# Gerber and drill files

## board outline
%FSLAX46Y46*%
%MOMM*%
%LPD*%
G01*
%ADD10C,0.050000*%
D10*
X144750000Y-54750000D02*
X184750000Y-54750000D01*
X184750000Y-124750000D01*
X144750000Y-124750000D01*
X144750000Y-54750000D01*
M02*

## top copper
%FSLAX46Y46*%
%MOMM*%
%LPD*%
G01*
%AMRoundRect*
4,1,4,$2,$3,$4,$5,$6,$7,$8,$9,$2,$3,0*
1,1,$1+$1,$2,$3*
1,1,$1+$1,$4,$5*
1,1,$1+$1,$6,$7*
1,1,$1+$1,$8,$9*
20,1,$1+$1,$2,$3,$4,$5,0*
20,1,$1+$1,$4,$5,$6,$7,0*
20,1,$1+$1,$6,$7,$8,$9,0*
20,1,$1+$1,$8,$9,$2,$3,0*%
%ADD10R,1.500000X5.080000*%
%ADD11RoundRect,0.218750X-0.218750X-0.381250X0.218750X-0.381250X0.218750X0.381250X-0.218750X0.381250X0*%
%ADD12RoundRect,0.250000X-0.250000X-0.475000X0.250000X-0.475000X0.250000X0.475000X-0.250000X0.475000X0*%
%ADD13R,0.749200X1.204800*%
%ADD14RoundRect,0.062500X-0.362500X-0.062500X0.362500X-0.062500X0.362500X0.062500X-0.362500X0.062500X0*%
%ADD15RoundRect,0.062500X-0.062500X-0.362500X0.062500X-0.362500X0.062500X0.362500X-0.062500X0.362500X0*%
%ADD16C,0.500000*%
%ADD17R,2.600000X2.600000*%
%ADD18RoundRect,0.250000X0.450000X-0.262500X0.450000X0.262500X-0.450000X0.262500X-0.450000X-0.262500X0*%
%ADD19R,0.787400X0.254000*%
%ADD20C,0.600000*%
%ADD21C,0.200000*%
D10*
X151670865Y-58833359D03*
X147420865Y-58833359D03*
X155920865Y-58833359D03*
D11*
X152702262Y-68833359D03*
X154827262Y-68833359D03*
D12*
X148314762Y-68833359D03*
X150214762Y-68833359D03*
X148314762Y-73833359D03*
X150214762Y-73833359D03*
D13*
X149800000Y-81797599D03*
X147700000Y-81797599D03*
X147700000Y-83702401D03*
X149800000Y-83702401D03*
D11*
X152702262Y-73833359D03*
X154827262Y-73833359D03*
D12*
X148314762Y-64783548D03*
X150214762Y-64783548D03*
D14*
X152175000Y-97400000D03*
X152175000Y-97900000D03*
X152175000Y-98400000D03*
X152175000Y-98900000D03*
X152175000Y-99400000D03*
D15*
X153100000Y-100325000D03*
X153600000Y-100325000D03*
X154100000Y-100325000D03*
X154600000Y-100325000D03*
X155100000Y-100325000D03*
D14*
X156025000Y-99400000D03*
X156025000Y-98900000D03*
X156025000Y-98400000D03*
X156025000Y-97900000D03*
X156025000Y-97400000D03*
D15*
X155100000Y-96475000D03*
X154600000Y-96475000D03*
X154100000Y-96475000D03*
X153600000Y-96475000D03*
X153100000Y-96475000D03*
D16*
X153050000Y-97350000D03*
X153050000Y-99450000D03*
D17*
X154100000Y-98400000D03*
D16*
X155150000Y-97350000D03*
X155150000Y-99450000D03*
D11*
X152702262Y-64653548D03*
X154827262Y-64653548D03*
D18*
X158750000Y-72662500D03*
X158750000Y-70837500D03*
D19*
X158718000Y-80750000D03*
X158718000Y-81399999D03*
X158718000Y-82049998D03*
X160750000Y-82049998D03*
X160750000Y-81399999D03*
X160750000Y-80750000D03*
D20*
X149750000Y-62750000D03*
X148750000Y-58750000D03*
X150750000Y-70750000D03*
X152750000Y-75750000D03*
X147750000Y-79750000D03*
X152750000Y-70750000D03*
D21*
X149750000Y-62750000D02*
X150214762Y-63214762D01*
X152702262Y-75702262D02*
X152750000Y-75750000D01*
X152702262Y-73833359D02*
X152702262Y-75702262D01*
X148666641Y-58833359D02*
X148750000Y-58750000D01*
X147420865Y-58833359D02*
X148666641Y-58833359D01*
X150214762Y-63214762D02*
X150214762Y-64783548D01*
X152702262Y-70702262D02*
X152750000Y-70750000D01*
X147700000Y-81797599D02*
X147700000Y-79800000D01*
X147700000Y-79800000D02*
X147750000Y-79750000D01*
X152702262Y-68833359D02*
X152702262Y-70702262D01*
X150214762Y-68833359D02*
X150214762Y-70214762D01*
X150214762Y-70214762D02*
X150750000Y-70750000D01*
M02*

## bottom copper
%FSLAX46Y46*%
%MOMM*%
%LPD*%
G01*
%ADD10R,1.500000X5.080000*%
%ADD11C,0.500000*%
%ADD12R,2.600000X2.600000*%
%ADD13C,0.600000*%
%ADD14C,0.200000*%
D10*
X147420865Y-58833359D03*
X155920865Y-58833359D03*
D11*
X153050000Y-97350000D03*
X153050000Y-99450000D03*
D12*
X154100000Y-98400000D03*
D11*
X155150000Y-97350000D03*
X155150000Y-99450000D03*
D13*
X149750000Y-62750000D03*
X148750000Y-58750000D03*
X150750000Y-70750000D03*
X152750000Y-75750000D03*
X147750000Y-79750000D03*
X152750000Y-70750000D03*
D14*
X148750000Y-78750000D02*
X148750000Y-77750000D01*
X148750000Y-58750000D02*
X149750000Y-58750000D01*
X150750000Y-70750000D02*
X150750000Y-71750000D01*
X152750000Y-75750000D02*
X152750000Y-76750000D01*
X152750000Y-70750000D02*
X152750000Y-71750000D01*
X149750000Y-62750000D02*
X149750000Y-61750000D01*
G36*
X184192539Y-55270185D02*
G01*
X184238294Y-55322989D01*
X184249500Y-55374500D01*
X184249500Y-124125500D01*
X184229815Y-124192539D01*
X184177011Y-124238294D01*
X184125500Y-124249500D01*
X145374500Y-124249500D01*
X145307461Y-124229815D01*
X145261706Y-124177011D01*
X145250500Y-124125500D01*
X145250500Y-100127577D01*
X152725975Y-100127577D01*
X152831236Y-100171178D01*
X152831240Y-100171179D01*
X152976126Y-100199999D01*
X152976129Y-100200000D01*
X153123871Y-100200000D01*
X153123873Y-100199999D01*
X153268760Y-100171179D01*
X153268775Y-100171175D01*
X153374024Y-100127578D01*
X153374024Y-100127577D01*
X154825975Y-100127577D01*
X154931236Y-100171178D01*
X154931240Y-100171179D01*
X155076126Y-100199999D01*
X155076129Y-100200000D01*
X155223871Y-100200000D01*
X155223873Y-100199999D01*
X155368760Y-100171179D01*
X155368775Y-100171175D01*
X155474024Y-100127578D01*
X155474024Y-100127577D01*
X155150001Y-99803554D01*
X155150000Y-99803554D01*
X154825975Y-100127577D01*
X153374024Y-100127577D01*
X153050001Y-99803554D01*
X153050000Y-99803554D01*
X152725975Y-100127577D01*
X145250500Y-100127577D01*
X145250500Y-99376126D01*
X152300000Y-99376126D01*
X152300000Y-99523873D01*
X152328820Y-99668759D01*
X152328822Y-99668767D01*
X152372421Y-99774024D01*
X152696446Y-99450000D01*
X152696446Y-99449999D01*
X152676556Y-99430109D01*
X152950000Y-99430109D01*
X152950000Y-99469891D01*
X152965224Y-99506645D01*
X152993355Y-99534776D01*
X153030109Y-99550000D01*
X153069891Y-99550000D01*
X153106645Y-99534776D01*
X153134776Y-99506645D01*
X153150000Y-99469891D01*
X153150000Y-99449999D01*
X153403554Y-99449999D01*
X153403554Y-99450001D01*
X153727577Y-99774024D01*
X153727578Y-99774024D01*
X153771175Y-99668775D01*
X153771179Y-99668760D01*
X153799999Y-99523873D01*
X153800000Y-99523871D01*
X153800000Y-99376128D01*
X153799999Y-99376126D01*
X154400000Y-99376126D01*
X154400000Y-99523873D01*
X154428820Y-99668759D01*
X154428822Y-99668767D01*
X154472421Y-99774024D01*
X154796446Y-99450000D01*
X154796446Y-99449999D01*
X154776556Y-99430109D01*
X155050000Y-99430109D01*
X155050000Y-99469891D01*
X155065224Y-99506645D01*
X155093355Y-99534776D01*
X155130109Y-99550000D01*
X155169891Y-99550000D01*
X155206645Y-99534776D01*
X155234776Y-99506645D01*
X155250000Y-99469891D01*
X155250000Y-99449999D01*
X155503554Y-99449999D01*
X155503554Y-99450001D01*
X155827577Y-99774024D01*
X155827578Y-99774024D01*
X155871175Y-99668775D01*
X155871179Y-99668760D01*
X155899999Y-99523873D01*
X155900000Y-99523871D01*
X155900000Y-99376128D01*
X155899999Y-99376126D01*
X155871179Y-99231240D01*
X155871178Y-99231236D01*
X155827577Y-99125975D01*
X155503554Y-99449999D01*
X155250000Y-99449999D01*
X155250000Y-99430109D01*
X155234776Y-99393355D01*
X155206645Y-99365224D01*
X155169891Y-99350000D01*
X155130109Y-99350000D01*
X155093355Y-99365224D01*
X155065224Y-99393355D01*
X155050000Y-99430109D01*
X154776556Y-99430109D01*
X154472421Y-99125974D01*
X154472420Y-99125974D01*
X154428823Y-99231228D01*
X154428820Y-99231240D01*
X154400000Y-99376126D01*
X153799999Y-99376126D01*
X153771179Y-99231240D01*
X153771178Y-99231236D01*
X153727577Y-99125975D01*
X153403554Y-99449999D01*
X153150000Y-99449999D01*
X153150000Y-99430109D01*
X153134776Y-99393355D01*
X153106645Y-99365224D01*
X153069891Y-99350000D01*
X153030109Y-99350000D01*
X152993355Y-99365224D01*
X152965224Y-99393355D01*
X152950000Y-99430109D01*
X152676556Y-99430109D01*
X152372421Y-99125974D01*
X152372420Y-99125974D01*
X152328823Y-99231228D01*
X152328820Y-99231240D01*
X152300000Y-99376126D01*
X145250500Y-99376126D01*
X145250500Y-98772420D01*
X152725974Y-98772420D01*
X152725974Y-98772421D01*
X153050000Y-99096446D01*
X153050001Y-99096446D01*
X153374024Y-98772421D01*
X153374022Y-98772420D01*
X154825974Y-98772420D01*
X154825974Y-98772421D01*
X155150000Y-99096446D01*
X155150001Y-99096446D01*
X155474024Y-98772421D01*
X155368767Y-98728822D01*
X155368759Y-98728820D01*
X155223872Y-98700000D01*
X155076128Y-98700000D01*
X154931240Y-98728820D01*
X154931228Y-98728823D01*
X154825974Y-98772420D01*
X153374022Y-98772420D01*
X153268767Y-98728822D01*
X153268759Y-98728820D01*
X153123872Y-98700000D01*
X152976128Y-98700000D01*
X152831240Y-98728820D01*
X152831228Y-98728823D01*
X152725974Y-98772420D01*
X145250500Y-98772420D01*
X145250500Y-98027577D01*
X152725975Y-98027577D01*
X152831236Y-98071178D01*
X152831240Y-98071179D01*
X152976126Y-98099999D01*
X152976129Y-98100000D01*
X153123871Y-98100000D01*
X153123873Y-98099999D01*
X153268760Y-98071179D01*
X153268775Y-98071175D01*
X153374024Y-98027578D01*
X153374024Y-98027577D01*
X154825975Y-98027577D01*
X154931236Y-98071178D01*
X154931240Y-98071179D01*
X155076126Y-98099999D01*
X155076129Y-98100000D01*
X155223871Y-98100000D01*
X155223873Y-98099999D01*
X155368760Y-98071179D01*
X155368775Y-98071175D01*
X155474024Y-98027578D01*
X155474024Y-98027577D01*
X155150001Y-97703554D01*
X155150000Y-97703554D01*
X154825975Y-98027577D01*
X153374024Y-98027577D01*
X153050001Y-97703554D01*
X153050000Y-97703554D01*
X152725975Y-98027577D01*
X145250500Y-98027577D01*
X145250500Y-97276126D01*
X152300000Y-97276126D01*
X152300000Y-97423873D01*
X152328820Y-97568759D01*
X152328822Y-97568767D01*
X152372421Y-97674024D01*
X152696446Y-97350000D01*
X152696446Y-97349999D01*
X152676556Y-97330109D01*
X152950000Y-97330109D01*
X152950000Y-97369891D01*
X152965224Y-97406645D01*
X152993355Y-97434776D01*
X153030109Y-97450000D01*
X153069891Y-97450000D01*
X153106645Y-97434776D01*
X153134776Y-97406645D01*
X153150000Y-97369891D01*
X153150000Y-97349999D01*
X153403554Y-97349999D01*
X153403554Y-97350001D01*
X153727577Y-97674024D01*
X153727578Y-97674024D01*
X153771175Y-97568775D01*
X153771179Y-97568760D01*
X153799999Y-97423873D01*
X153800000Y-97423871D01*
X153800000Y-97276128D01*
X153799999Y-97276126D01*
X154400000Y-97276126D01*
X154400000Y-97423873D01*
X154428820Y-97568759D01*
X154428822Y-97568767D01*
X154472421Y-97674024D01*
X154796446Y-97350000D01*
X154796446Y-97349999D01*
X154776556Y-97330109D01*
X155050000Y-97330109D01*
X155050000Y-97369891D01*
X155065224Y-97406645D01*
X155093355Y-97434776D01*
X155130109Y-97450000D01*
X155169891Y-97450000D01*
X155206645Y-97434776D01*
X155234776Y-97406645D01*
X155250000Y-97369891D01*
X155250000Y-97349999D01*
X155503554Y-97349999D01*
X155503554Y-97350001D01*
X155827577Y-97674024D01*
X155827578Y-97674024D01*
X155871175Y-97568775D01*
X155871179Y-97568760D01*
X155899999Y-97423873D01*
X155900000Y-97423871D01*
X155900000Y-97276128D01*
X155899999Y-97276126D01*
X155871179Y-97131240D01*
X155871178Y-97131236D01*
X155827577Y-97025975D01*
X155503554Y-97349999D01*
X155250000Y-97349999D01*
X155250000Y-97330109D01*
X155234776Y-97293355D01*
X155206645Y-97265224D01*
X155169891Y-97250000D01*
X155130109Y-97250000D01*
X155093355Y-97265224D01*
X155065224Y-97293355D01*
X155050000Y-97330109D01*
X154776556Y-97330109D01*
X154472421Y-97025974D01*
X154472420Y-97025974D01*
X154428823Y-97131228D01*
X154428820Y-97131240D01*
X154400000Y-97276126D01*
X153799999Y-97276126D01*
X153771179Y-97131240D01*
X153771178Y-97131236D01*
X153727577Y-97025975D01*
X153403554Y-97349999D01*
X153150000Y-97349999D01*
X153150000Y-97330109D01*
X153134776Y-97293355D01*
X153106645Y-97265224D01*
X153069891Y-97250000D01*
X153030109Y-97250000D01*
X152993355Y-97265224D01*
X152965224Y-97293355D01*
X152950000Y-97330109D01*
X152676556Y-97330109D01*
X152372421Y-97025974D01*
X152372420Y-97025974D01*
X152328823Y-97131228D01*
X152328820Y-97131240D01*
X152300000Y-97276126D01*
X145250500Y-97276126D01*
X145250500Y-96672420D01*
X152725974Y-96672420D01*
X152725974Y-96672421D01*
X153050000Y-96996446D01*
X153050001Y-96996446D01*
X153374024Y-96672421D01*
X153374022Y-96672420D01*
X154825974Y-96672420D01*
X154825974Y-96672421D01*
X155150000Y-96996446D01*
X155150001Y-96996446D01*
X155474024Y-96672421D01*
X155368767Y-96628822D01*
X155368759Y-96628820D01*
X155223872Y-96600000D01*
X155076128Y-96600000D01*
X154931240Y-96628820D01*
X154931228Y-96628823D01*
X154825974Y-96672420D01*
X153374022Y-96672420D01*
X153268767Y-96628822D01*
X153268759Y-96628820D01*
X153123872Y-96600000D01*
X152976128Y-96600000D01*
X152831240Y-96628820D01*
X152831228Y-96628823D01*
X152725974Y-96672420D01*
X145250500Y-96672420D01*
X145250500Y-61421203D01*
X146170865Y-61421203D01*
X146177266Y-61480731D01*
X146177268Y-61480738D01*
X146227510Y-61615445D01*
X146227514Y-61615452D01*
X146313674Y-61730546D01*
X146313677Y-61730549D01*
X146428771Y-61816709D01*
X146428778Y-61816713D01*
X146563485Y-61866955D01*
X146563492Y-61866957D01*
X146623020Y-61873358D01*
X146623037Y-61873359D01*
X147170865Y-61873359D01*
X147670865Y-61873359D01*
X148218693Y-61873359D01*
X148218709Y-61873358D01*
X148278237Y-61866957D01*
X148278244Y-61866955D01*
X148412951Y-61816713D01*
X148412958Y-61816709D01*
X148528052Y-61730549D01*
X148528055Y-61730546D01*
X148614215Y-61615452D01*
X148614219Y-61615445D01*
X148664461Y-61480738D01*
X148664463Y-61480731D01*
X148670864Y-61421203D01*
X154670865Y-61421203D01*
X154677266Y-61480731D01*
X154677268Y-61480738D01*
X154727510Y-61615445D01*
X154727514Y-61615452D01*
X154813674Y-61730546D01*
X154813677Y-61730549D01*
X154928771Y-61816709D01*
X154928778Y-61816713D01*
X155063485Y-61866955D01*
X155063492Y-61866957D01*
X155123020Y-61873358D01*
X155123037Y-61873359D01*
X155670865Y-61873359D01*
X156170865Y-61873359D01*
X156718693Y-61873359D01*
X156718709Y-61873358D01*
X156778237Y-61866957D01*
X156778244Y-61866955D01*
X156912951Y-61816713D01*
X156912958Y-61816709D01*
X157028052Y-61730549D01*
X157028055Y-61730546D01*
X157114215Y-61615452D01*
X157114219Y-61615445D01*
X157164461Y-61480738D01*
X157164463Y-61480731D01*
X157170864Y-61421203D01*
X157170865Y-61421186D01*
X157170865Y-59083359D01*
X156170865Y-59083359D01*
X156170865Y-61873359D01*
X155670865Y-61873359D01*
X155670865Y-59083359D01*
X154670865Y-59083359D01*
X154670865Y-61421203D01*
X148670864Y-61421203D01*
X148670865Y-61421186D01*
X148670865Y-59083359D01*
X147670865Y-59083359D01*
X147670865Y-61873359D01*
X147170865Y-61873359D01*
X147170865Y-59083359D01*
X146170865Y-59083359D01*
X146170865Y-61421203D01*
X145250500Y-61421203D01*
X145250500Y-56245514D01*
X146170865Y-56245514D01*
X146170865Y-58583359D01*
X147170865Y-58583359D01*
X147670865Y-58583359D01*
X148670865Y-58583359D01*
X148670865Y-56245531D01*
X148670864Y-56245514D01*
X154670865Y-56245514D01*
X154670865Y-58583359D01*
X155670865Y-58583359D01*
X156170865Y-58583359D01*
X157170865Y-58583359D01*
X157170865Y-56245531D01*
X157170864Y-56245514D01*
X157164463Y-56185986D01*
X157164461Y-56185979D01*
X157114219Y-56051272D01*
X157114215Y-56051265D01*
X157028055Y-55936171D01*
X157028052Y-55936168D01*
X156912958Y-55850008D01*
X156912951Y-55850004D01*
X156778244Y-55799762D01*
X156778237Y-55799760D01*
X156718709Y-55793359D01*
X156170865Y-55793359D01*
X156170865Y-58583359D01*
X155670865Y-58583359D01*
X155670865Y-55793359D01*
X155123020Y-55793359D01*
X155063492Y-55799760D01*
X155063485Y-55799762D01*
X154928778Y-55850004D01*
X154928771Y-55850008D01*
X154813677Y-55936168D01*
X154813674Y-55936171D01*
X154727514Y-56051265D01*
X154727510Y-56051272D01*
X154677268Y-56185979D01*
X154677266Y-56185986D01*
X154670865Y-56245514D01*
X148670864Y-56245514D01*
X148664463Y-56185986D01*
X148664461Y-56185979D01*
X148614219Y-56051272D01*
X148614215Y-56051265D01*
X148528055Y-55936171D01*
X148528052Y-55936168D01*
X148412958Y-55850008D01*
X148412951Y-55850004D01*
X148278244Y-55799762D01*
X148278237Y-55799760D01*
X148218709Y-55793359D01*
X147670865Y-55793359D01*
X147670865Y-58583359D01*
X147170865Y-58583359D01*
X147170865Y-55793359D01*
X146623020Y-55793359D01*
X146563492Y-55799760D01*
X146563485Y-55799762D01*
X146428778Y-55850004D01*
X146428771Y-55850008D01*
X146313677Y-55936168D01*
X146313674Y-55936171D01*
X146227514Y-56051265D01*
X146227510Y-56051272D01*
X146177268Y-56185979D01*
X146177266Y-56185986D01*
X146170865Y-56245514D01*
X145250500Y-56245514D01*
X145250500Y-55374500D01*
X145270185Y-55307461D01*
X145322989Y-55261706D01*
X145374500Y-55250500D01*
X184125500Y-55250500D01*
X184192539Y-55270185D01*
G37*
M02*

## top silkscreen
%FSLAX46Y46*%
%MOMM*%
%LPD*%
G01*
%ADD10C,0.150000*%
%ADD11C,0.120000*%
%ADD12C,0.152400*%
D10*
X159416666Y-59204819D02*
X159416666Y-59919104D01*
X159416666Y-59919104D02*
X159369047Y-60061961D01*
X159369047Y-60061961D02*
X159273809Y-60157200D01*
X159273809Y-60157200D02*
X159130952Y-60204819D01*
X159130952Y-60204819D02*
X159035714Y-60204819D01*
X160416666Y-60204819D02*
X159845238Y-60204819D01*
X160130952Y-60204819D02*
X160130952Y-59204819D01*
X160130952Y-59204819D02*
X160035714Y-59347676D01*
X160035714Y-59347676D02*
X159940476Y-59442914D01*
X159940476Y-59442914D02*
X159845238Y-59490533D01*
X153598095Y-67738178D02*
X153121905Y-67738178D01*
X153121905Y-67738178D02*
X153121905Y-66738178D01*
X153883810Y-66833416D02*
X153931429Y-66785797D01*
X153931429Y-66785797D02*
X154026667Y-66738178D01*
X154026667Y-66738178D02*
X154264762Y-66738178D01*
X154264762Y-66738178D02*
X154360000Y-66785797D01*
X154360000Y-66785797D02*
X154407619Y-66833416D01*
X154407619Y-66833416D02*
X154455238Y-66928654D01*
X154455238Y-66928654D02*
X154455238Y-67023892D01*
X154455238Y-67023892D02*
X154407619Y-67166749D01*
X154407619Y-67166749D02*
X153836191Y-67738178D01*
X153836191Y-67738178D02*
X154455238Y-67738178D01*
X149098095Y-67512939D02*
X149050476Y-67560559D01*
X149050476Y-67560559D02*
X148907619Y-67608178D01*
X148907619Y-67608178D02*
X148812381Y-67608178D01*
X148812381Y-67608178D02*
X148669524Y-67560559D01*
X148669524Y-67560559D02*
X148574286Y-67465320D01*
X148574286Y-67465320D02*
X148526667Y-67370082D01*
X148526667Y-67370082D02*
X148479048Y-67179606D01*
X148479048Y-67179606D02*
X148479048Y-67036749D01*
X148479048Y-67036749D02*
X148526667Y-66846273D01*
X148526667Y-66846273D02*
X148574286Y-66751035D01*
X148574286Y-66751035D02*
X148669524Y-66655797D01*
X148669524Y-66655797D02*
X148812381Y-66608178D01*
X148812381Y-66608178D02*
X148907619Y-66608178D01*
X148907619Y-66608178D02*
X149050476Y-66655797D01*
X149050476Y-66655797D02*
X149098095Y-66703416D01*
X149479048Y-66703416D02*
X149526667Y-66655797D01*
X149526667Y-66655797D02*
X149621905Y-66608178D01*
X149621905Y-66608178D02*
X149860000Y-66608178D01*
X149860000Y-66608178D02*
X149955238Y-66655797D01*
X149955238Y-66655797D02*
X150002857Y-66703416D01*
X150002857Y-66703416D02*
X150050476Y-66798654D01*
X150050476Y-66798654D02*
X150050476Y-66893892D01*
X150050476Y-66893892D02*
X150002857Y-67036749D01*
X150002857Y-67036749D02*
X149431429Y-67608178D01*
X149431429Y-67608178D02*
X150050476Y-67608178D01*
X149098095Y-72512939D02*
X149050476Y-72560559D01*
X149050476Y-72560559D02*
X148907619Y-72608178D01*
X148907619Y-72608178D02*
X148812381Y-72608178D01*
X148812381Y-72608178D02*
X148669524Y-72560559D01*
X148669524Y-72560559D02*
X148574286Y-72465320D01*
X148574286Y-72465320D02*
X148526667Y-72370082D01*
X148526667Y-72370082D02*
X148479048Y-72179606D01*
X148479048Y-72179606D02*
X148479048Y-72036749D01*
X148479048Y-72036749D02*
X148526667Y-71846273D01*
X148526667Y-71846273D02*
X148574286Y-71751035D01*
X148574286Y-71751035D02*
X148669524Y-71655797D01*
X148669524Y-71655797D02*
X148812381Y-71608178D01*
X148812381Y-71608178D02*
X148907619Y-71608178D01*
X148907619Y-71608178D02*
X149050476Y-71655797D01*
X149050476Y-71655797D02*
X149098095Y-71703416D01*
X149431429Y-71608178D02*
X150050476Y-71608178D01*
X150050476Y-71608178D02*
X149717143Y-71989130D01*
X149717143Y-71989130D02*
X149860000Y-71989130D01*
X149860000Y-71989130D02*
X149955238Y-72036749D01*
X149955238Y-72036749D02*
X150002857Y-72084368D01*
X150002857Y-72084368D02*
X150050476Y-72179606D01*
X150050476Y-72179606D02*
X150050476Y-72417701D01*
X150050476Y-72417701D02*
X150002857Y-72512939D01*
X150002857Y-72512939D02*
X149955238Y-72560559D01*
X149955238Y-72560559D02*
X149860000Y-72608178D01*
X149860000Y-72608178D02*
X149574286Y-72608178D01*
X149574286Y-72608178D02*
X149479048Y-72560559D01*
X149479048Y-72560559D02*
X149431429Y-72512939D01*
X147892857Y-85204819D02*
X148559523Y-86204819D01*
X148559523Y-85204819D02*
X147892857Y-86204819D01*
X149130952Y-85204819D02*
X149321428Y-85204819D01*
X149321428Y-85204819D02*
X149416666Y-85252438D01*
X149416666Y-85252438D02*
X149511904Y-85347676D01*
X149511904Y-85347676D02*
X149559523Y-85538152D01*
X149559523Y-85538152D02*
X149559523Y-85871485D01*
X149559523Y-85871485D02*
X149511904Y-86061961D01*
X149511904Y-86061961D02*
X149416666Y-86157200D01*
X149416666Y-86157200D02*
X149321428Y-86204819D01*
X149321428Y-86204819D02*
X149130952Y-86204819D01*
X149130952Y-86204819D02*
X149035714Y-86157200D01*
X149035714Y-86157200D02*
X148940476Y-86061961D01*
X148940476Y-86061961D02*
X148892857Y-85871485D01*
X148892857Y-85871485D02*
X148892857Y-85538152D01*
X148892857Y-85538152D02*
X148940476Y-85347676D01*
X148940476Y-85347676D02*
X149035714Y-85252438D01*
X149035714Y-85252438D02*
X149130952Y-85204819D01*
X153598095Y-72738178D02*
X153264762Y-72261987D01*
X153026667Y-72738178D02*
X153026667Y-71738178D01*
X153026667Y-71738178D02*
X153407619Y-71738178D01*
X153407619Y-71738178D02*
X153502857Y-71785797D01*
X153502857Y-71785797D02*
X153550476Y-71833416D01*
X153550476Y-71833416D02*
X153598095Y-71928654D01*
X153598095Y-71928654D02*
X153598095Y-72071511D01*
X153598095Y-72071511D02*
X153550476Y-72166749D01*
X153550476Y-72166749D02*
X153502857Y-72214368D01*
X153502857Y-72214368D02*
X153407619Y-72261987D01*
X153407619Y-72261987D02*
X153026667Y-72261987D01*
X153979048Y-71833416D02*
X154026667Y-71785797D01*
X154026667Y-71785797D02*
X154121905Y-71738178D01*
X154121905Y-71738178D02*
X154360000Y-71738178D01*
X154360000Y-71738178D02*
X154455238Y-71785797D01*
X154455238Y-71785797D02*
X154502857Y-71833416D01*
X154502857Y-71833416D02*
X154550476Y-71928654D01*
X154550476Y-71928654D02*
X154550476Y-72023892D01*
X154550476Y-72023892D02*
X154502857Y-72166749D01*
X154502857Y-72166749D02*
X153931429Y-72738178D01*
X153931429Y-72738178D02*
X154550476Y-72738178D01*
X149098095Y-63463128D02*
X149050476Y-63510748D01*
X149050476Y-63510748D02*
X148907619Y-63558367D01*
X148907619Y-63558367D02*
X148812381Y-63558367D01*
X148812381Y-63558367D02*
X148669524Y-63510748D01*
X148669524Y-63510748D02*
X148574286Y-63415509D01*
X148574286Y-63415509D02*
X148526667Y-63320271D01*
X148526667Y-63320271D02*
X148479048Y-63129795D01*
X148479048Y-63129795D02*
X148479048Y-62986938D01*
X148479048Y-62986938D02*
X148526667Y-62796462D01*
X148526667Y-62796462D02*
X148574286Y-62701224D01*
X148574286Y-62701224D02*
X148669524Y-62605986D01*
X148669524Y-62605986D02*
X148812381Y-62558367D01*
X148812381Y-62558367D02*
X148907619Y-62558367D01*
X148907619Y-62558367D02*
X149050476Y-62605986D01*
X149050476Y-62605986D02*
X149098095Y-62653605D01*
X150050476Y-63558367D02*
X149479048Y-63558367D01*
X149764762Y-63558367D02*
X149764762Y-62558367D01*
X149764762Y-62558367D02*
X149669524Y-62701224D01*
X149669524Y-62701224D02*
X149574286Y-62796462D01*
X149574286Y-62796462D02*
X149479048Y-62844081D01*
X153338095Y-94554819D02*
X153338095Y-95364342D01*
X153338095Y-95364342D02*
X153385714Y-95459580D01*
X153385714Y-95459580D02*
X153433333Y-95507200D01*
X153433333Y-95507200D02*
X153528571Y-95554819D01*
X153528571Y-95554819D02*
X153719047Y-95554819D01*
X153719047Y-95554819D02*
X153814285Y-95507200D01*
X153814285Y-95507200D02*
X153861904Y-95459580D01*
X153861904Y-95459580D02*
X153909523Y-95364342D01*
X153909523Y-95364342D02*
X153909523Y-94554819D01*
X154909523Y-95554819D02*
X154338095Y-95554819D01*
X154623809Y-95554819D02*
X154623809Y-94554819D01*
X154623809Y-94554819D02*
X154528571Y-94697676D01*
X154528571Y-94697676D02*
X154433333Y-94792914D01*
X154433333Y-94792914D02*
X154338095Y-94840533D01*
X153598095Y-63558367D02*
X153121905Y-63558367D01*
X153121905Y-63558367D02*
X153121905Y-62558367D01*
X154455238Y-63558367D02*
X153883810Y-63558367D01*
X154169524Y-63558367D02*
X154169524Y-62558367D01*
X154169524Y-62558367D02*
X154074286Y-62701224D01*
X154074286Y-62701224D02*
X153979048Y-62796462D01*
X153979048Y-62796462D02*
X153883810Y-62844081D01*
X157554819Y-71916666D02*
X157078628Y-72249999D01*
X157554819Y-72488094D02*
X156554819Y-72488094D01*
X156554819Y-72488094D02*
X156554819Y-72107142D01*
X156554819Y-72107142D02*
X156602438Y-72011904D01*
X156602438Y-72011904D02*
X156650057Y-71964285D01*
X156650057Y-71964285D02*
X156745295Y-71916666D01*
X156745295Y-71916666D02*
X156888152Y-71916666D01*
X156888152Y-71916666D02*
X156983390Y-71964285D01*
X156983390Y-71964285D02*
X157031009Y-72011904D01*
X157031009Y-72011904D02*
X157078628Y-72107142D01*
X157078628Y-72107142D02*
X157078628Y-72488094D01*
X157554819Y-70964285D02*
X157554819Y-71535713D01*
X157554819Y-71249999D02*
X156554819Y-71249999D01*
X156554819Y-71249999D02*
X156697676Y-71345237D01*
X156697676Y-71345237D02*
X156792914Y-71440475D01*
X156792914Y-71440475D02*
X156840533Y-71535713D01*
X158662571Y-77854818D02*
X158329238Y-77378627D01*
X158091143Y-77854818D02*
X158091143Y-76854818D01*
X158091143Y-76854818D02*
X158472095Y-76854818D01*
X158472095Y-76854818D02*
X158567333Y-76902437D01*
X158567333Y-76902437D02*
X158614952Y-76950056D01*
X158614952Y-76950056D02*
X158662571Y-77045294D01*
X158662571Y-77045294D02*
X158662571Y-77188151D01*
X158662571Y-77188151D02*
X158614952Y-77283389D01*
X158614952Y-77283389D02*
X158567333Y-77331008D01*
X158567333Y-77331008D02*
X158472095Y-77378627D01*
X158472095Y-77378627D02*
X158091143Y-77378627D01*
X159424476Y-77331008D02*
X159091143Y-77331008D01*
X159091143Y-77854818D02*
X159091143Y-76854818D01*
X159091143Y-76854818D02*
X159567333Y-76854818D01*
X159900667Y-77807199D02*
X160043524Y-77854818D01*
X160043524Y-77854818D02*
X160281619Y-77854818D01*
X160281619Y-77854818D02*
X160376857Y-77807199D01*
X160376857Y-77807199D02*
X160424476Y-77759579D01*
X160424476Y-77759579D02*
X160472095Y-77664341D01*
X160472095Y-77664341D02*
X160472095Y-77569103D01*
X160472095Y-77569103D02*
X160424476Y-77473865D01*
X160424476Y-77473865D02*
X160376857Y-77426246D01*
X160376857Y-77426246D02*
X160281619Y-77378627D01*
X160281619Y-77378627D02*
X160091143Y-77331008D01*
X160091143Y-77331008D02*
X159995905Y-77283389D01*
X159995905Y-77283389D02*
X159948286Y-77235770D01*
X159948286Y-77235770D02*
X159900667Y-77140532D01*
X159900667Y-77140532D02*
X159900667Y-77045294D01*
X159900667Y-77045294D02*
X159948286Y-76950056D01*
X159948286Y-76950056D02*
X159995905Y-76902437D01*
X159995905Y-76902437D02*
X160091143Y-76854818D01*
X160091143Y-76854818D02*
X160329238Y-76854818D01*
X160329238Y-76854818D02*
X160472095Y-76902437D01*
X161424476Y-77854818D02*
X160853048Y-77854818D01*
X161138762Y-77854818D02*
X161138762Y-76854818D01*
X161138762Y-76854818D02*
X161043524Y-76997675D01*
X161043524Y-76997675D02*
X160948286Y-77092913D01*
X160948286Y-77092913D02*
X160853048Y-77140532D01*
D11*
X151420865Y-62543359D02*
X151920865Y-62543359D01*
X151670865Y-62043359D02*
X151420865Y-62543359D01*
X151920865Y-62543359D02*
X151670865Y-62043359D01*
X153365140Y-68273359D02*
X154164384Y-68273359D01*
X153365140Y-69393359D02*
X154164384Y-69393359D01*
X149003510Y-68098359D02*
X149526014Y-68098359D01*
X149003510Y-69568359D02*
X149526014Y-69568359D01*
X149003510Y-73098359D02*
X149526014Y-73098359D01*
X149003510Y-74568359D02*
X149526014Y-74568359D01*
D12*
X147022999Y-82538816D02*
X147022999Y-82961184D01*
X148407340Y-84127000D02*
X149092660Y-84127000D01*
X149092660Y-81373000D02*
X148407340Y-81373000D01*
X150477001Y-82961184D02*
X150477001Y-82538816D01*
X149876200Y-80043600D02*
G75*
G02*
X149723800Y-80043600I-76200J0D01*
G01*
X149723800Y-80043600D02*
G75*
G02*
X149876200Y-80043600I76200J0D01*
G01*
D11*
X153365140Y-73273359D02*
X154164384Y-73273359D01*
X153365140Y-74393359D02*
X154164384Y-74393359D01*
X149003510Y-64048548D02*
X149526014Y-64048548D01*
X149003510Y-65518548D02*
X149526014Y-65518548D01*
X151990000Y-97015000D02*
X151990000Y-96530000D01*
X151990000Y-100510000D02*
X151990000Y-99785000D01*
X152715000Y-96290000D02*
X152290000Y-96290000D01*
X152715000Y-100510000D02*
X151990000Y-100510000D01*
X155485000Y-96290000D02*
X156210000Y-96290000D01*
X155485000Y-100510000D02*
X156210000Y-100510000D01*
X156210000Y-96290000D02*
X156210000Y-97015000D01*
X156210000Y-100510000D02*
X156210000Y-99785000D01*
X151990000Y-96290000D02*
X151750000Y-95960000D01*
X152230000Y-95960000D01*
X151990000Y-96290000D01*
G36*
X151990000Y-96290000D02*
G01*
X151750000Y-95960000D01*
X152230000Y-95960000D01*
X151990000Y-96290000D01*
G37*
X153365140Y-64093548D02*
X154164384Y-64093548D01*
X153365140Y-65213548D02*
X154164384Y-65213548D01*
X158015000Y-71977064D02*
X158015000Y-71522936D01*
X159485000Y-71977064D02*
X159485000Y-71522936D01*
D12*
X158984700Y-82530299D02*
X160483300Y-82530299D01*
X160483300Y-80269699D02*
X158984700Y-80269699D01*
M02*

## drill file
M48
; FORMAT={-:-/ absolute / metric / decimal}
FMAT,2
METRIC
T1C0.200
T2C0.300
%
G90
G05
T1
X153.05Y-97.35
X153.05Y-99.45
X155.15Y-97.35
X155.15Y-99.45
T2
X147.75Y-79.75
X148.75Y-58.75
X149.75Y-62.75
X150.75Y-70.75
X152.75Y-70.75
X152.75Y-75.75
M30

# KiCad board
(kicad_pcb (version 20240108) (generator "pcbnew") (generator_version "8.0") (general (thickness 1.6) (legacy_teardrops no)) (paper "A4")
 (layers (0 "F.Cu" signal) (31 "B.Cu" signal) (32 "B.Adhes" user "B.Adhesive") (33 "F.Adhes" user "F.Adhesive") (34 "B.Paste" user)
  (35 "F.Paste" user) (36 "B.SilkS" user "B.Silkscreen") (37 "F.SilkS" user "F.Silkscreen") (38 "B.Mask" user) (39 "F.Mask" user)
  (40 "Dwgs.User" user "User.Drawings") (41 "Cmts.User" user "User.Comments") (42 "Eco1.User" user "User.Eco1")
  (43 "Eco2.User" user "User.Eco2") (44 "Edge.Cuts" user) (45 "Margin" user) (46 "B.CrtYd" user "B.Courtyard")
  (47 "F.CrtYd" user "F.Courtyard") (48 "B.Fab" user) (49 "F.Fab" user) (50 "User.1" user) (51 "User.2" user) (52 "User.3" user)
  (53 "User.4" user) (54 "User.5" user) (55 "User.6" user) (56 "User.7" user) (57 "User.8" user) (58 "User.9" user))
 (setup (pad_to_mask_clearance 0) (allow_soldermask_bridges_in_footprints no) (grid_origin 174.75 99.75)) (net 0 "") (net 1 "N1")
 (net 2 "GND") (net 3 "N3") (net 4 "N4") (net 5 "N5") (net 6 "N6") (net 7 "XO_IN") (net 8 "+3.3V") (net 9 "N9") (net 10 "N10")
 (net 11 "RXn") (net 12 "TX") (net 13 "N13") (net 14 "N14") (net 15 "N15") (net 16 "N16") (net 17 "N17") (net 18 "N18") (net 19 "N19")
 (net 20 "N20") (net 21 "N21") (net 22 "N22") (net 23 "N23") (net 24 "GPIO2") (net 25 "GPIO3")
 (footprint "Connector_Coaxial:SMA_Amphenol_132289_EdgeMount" (layer "F.Cu") (at 151.670865 58.833359 90)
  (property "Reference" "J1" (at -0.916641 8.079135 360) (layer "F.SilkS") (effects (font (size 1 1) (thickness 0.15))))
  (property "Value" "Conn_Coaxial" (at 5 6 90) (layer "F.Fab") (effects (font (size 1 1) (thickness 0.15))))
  (fp_line (start -3.71 -0.25) (end -3.71 0.25) (stroke (width 0.12) (type solid)) (layer "F.SilkS"))
  (fp_line (start -3.21 0) (end -3.71 -0.25) (stroke (width 0.12) (type solid)) (layer "F.SilkS"))
  (fp_line (start -3.71 0.25) (end -3.21 0) (stroke (width 0.12) (type solid)) (layer "F.SilkS"))
  (pad "1" smd rect (at 0 0 180) (size 1.5 5.08) (layers "F.Cu" "F.Paste" "F.Mask") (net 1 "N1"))
  (pad "2" smd rect (at 0 -4.25 180) (size 1.5 5.08) (layers "F.Cu" "F.Paste" "F.Mask") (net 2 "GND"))
  (pad "2" smd rect (at 0 -4.25 180) (size 1.5 5.08) (layers "B.Cu" "B.Paste" "B.Mask") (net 2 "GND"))
  (pad "2" smd rect (at 0 4.25 180) (size 1.5 5.08) (layers "F.Cu" "F.Paste" "F.Mask") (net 2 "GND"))
  (pad "2" smd rect (at 0 4.25 180) (size 1.5 5.08) (layers "B.Cu" "B.Paste" "B.Mask") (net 2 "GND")))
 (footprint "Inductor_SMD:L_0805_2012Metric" (layer "F.Cu") (at 153.764762 68.833359)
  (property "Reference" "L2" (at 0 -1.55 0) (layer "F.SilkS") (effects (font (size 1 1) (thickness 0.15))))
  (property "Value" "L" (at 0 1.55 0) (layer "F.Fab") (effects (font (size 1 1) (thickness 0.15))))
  (fp_line (start -0.399622 -0.56) (end 0.399622 -0.56) (stroke (width 0.12) (type solid)) (layer "F.SilkS"))
  (fp_line (start -0.399622 0.56) (end 0.399622 0.56) (stroke (width 0.12) (type solid)) (layer "F.SilkS"))
  (pad "1" smd roundrect (at -1.0625 0) (size 0.875 1.2) (layers "F.Cu" "F.Paste" "F.Mask") (roundrect_rratio 0.25) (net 2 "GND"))
  (pad "2" smd roundrect (at 1.0625 0) (size 0.875 1.2) (layers "F.Cu" "F.Paste" "F.Mask") (roundrect_rratio 0.25) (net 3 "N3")))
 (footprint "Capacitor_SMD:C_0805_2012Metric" (layer "F.Cu") (at 149.264762 68.833359)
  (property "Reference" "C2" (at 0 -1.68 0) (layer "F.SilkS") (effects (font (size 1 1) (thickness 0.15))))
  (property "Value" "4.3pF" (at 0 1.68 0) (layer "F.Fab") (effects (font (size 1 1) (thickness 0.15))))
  (fp_line (start -0.261252 -0.735) (end 0.261252 -0.735) (stroke (width 0.12) (type solid)) (layer "F.SilkS"))
  (fp_line (start -0.261252 0.735) (end 0.261252 0.735) (stroke (width 0.12) (type solid)) (layer "F.SilkS"))
  (pad "1" smd roundrect (at -0.95 0) (size 1 1.45) (layers "F.Cu" "F.Paste" "F.Mask") (roundrect_rratio 0.25) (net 1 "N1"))
  (pad "2" smd roundrect (at 0.95 0) (size 1 1.45) (layers "F.Cu" "F.Paste" "F.Mask") (roundrect_rratio 0.25) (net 2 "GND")))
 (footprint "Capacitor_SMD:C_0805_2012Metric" (layer "F.Cu") (at 149.264762 73.833359)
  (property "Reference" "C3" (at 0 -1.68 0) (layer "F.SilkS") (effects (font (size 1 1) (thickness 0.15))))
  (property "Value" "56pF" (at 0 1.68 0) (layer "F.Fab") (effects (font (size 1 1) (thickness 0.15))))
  (fp_line (start -0.261252 -0.735) (end 0.261252 -0.735) (stroke (width 0.12) (type solid)) (layer "F.SilkS"))
  (fp_line (start -0.261252 0.735) (end 0.261252 0.735) (stroke (width 0.12) (type solid)) (layer "F.SilkS"))
  (pad "1" smd roundrect (at -0.95 0) (size 1 1.45) (layers "F.Cu" "F.Paste" "F.Mask") (roundrect_rratio 0.25) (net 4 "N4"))
  (pad "2" smd roundrect (at 0.95 0) (size 1 1.45) (layers "F.Cu" "F.Paste" "F.Mask") (roundrect_rratio 0.25) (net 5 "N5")))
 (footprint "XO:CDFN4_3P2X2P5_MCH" (layer "F.Cu") (at 148.75 82.75 -90)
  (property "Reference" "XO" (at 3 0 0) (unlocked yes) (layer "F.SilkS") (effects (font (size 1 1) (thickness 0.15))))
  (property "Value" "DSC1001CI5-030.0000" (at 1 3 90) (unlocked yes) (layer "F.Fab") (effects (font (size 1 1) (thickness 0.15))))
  (fp_line (start -0.211184 1.727001) (end 0.211184 1.727001) (stroke (width 0.1524) (type solid)) (layer "F.SilkS"))
  (fp_line (start 1.377 0.34266) (end 1.377 -0.34266) (stroke (width 0.1524) (type solid)) (layer "F.SilkS"))
  (fp_line (start -1.377 -0.34266) (end -1.377 0.34266) (stroke (width 0.1524) (type solid)) (layer "F.SilkS"))
  (fp_line (start 0.211184 -1.727001) (end -0.211184 -1.727001) (stroke (width 0.1524) (type solid)) (layer "F.SilkS"))
  (fp_circle (center -2.7064 -1.05) (end -2.6302 -1.05) (stroke (width 0.1524) (type solid)) (fill none) (layer "F.SilkS"))
  (pad "1" smd rect (at -0.952401 -1.05 270) (size 1.2048 0.7492) (layers "F.Cu" "F.Paste" "F.Mask") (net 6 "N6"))
  (pad "2" smd rect (at -0.952401 1.05 270) (size 1.2048 0.7492) (layers "F.Cu" "F.Paste" "F.Mask") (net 2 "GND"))
  (pad "3" smd rect (at 0.952401 1.05 270) (size 1.2048 0.7492) (layers "F.Cu" "F.Paste" "F.Mask") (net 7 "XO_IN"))
  (pad "4" smd rect (at 0.952401 -1.05 270) (size 1.2048 0.7492) (layers "F.Cu" "F.Paste" "F.Mask") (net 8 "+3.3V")))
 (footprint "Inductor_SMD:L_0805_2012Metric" (layer "F.Cu") (at 153.764762 73.833359)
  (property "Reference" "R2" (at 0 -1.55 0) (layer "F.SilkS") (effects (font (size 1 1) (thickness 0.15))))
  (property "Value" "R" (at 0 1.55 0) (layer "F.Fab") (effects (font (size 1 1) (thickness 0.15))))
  (fp_line (start -0.399622 -0.56) (end 0.399622 -0.56) (stroke (width 0.12) (type solid)) (layer "F.SilkS"))
  (fp_line (start -0.399622 0.56) (end 0.399622 0.56) (stroke (width 0.12) (type solid)) (layer "F.SilkS"))
  (pad "1" smd roundrect (at -1.0625 0) (size 0.875 1.2) (layers "F.Cu" "F.Paste" "F.Mask") (roundrect_rratio 0.25) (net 2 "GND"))
  (pad "2" smd roundrect (at 1.0625 0) (size 0.875 1.2) (layers "F.Cu" "F.Paste" "F.Mask") (roundrect_rratio 0.25) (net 4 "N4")))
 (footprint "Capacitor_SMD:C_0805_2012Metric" (layer "F.Cu") (at 149.264762 64.783548)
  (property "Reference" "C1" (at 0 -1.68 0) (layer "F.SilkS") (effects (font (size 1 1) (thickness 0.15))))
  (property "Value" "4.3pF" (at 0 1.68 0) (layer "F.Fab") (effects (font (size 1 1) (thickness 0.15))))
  (fp_line (start -0.261252 -0.735) (end 0.261252 -0.735) (stroke (width 0.12) (type solid)) (layer "F.SilkS"))
  (fp_line (start -0.261252 0.735) (end 0.261252 0.735) (stroke (width 0.12) (type solid)) (layer "F.SilkS"))
  (pad "1" smd roundrect (at -0.95 0) (size 1 1.45) (layers "F.Cu" "F.Paste" "F.Mask") (roundrect_rratio 0.25) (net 5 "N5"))
  (pad "2" smd roundrect (at 0.95 0) (size 1 1.45) (layers "F.Cu" "F.Paste" "F.Mask") (roundrect_rratio 0.25) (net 2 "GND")))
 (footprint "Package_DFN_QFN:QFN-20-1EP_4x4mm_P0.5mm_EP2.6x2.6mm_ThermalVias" (layer "F.Cu") (at 154.1 98.4)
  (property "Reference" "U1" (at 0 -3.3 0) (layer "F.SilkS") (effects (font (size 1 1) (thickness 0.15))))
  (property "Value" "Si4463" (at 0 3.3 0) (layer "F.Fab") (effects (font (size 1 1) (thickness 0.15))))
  (fp_line (start -2.11 -1.385) (end -2.11 -1.87) (stroke (width 0.12) (type solid)) (layer "F.SilkS"))
  (fp_line (start -2.11 2.11) (end -2.11 1.385) (stroke (width 0.12) (type solid)) (layer "F.SilkS"))
  (fp_line (start -1.385 -2.11) (end -1.81 -2.11) (stroke (width 0.12) (type solid)) (layer "F.SilkS"))
  (fp_line (start -1.385 2.11) (end -2.11 2.11) (stroke (width 0.12) (type solid)) (layer "F.SilkS"))
  (fp_line (start 1.385 -2.11) (end 2.11 -2.11) (stroke (width 0.12) (type solid)) (layer "F.SilkS"))
  (fp_line (start 1.385 2.11) (end 2.11 2.11) (stroke (width 0.12) (type solid)) (layer "F.SilkS"))
  (fp_line (start 2.11 -2.11) (end 2.11 -1.385) (stroke (width 0.12) (type solid)) (layer "F.SilkS"))
  (fp_line (start 2.11 2.11) (end 2.11 1.385) (stroke (width 0.12) (type solid)) (layer "F.SilkS"))
  (fp_poly
   (pts (xy -2.11 -2.11) (xy -2.35 -2.44) (xy -1.87 -2.44) (xy -2.11 -2.11)) (stroke (width 0.12) (type solid)) (fill solid)
   (layer "F.SilkS"))
  (pad "" smd roundrect (at -0.65 -0.65) (size 1.13 1.13) (layers "F.Paste") (roundrect_rratio 0.221239))
  (pad "" smd roundrect (at -0.65 0.65) (size 1.13 1.13) (layers "F.Paste") (roundrect_rratio 0.221239))
  (pad "" smd roundrect (at 0.65 -0.65) (size 1.13 1.13) (layers "F.Paste") (roundrect_rratio 0.221239))
  (pad "" smd roundrect (at 0.65 0.65) (size 1.13 1.13) (layers "F.Paste") (roundrect_rratio 0.221239))
  (pad "1" smd roundrect (at -1.925 -1) (size 0.85 0.25) (layers "F.Cu" "F.Paste" "F.Mask") (roundrect_rratio 0.25) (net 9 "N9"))
  (pad "2" smd roundrect (at -1.925 -0.5) (size 0.85 0.25) (layers "F.Cu" "F.Paste" "F.Mask") (roundrect_rratio 0.25) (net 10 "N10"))
  (pad "3" smd roundrect (at -1.925 0) (size 0.85 0.25) (layers "F.Cu" "F.Paste" "F.Mask") (roundrect_rratio 0.25) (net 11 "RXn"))
  (pad "4" smd roundrect (at -1.925 0.5) (size 0.85 0.25) (layers "F.Cu" "F.Paste" "F.Mask") (roundrect_rratio 0.25) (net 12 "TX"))
  (pad "5" smd roundrect (at -1.925 1) (size 0.85 0.25) (layers "F.Cu" "F.Paste" "F.Mask") (roundrect_rratio 0.25) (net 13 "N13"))
  (pad "6" smd roundrect (at -1 1.925) (size 0.25 0.85) (layers "F.Cu" "F.Paste" "F.Mask") (roundrect_rratio 0.25) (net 8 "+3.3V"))
  (pad "7" smd roundrect (at -0.5 1.925) (size 0.25 0.85) (layers "F.Cu" "F.Paste" "F.Mask") (roundrect_rratio 0.25) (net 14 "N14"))
  (pad "8" smd roundrect (at 0 1.925) (size 0.25 0.85) (layers "F.Cu" "F.Paste" "F.Mask") (roundrect_rratio 0.25) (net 8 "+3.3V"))
  (pad "9" smd roundrect (at 0.5 1.925) (size 0.25 0.85) (layers "F.Cu" "F.Paste" "F.Mask") (roundrect_rratio 0.25) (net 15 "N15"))
  (pad "10" smd roundrect (at 1 1.925) (size 0.25 0.85) (layers "F.Cu" "F.Paste" "F.Mask") (roundrect_rratio 0.25) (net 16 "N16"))
  (pad "11" smd roundrect (at 1.925 1) (size 0.85 0.25) (layers "F.Cu" "F.Paste" "F.Mask") (roundrect_rratio 0.25) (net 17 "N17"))
  (pad "12" smd roundrect (at 1.925 0.5) (size 0.85 0.25) (layers "F.Cu" "F.Paste" "F.Mask") (roundrect_rratio 0.25) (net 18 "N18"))
  (pad "13" smd roundrect (at 1.925 0) (size 0.85 0.25) (layers "F.Cu" "F.Paste" "F.Mask") (roundrect_rratio 0.25) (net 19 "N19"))
  (pad "14" smd roundrect (at 1.925 -0.5) (size 0.85 0.25) (layers "F.Cu" "F.Paste" "F.Mask") (roundrect_rratio 0.25) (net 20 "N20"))
  (pad "15" smd roundrect (at 1.925 -1) (size 0.85 0.25) (layers "F.Cu" "F.Paste" "F.Mask") (roundrect_rratio 0.25) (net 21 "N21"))
  (pad "16" smd roundrect (at 1 -1.925) (size 0.25 0.85) (layers "F.Cu" "F.Paste" "F.Mask") (roundrect_rratio 0.25) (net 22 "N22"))
  (pad "17" smd roundrect (at 0.5 -1.925) (size 0.25 0.85) (layers "F.Cu" "F.Paste" "F.Mask") (roundrect_rratio 0.25) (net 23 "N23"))
  (pad "18" smd roundrect (at 0 -1.925) (size 0.25 0.85) (layers "F.Cu" "F.Paste" "F.Mask") (roundrect_rratio 0.25) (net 2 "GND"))
  (pad "19" smd roundrect (at -0.5 -1.925) (size 0.25 0.85) (layers "F.Cu" "F.Paste" "F.Mask") (roundrect_rratio 0.25) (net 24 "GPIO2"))
  (pad "20" smd roundrect (at -1 -1.925) (size 0.25 0.85) (layers "F.Cu" "F.Paste" "F.Mask") (roundrect_rratio 0.25) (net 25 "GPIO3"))
  (pad "21" thru_hole circle (at -1.05 -1.05) (size 0.5 0.5) (drill 0.2) (layers "*.Cu") (remove_unused_layers no) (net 2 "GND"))
  (pad "21" thru_hole circle (at -1.05 1.05) (size 0.5 0.5) (drill 0.2) (layers "*.Cu") (remove_unused_layers no) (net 2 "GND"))
  (pad "21" smd rect (at 0 0) (size 2.6 2.6) (layers "F.Cu" "F.Mask") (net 2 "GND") (zone_connect 2))
  (pad "21" smd rect (at 0 0) (size 2.6 2.6) (layers "B.Cu") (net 2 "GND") (zone_connect 2))
  (pad "21" thru_hole circle (at 1.05 -1.05) (size 0.5 0.5) (drill 0.2) (layers "*.Cu") (remove_unused_layers no) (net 2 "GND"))
  (pad "21" thru_hole circle (at 1.05 1.05) (size 0.5 0.5) (drill 0.2) (layers "*.Cu") (remove_unused_layers no) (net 2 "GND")))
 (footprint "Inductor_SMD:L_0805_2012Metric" (layer "F.Cu") (at 153.764762 64.653548)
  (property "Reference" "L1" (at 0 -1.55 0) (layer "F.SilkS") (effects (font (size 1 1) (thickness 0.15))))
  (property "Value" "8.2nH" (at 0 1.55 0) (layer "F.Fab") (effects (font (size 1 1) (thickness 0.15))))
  (fp_line (start -0.399622 -0.56) (end 0.399622 -0.56) (stroke (width 0.12) (type solid)) (layer "F.SilkS"))
  (fp_line (start -0.399622 0.56) (end 0.399622 0.56) (stroke (width 0.12) (type solid)) (layer "F.SilkS"))
  (pad "1" smd roundrect (at -1.0625 0) (size 0.875 1.2) (layers "F.Cu" "F.Paste" "F.Mask") (roundrect_rratio 0.25) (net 5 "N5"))
  (pad "2" smd roundrect (at 1.0625 0) (size 0.875 1.2) (layers "F.Cu" "F.Paste" "F.Mask") (roundrect_rratio 0.25) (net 1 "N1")))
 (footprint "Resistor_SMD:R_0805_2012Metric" (layer "F.Cu") (at 158.75 71.75 90)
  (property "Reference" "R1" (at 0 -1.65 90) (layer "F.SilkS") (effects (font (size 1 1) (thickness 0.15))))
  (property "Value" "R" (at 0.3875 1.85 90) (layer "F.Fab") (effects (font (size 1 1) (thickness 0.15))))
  (fp_line (start -0.227064 -0.735) (end 0.227064 -0.735) (stroke (width 0.12) (type solid)) (layer "F.SilkS"))
  (fp_line (start -0.227064 0.735) (end 0.227064 0.735) (stroke (width 0.12) (type solid)) (layer "F.SilkS"))
  (pad "1" smd roundrect (at -0.9125 0 90) (size 1.025 1.4) (layers "F.Cu" "F.Paste" "F.Mask") (roundrect_rratio 0.243902) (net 4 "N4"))
  (pad "2" smd roundrect (at 0.9125 0 90) (size 1.025 1.4) (layers "F.Cu" "F.Paste" "F.Mask") (roundrect_rratio 0.243902) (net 3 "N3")))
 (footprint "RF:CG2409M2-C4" (layer "F.Cu") (at 159.734 81.399999)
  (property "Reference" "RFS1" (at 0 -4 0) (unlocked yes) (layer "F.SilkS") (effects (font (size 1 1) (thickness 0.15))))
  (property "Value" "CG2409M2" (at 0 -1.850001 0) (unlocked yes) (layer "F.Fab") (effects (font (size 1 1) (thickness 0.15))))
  (fp_line (start -0.7493 1.1303) (end 0.7493 1.1303) (stroke (width 0.1524) (type solid)) (layer "F.SilkS"))
  (fp_line (start 0.7493 -1.1303) (end -0.7493 -1.1303) (stroke (width 0.1524) (type solid)) (layer "F.SilkS"))
  (pad "1" smd rect (at -1.016 -0.649999) (size 0.7874 0.254) (layers "F.Cu" "F.Paste" "F.Mask") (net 11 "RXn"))
  (pad "2" smd rect (at -1.016 0) (size 0.7874 0.254) (layers "F.Cu" "F.Paste" "F.Mask") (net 2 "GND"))
  (pad "3" smd rect (at -1.016 0.649999) (size 0.7874 0.254) (layers "F.Cu" "F.Paste" "F.Mask") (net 12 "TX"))
  (pad "4" smd rect (at 1.016 0.649999) (size 0.7874 0.254) (layers "F.Cu" "F.Paste" "F.Mask") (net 24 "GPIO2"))
  (pad "5" smd rect (at 1.016 0) (size 0.7874 0.254) (layers "F.Cu" "F.Paste" "F.Mask") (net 3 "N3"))
  (pad "6" smd rect (at 1.016 -0.649999) (size 0.7874 0.254) (layers "F.Cu" "F.Paste" "F.Mask") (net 25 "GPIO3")))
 (gr_rect (start 144.75 54.75) (end 184.75 124.75) (stroke (width 0.05) (type default)) (fill none) (layer "Edge.Cuts"))
 (segment (start 149.75 62.75) (end 150.214762 63.214762) (width 0.2) (layer "F.Cu") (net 2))
 (segment (start 152.702262 75.702262) (end 152.75 75.75) (width 0.2) (layer "F.Cu") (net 2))
 (segment (start 152.702262 73.833359) (end 152.702262 75.702262) (width 0.2) (layer "F.Cu") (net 2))
 (segment (start 148.666641 58.833359) (end 148.75 58.75) (width 0.2) (layer "F.Cu") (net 2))
 (segment (start 147.420865 58.833359) (end 148.666641 58.833359) (width 0.2) (layer "F.Cu") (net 2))
 (segment (start 150.214762 63.214762) (end 150.214762 64.783548) (width 0.2) (layer "F.Cu") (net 2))
 (segment (start 152.702262 70.702262) (end 152.75 70.75) (width 0.2) (layer "F.Cu") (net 2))
 (segment (start 147.7 81.797599) (end 147.7 79.8) (width 0.2) (layer "F.Cu") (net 2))
 (segment (start 147.7 79.8) (end 147.75 79.75) (width 0.2) (layer "F.Cu") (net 2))
 (segment (start 152.702262 68.833359) (end 152.702262 70.702262) (width 0.2) (layer "F.Cu") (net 2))
 (segment (start 150.214762 68.833359) (end 150.214762 70.214762) (width 0.2) (layer "F.Cu") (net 2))
 (segment (start 150.214762 70.214762) (end 150.75 70.75) (width 0.2) (layer "F.Cu") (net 2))
 (via (at 149.75 62.75) (size 0.6) (drill 0.3) (layers "F.Cu" "B.Cu") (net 2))
 (via (at 148.75 58.75) (size 0.6) (drill 0.3) (layers "F.Cu" "B.Cu") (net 2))
 (via (at 150.75 70.75) (size 0.6) (drill 0.3) (layers "F.Cu" "B.Cu") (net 2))
 (via (at 152.75 75.75) (size 0.6) (drill 0.3) (layers "F.Cu" "B.Cu") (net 2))
 (via (at 147.75 79.75) (size 0.6) (drill 0.3) (layers "F.Cu" "B.Cu") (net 2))
 (via (at 152.75 70.75) (size 0.6) (drill 0.3) (layers "F.Cu" "B.Cu") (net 2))
 (segment (start 148.75 78.75) (end 148.75 77.75) (width 0.2) (layer "B.Cu") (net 2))
 (segment (start 148.75 58.75) (end 149.75 58.75) (width 0.2) (layer "B.Cu") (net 2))
 (segment (start 150.75 70.75) (end 150.75 71.75) (width 0.2) (layer "B.Cu") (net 2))
 (segment (start 152.75 75.75) (end 152.75 76.75) (width 0.2) (layer "B.Cu") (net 2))
 (segment (start 152.75 70.75) (end 152.75 71.75) (width 0.2) (layer "B.Cu") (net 2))
 (segment (start 149.75 62.75) (end 149.75 61.75) (width 0.2) (layer "B.Cu") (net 2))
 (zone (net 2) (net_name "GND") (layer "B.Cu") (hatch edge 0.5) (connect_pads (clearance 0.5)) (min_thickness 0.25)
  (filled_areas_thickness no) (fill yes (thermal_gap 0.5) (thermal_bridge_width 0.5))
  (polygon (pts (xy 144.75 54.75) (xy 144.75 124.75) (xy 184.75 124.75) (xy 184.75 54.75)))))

